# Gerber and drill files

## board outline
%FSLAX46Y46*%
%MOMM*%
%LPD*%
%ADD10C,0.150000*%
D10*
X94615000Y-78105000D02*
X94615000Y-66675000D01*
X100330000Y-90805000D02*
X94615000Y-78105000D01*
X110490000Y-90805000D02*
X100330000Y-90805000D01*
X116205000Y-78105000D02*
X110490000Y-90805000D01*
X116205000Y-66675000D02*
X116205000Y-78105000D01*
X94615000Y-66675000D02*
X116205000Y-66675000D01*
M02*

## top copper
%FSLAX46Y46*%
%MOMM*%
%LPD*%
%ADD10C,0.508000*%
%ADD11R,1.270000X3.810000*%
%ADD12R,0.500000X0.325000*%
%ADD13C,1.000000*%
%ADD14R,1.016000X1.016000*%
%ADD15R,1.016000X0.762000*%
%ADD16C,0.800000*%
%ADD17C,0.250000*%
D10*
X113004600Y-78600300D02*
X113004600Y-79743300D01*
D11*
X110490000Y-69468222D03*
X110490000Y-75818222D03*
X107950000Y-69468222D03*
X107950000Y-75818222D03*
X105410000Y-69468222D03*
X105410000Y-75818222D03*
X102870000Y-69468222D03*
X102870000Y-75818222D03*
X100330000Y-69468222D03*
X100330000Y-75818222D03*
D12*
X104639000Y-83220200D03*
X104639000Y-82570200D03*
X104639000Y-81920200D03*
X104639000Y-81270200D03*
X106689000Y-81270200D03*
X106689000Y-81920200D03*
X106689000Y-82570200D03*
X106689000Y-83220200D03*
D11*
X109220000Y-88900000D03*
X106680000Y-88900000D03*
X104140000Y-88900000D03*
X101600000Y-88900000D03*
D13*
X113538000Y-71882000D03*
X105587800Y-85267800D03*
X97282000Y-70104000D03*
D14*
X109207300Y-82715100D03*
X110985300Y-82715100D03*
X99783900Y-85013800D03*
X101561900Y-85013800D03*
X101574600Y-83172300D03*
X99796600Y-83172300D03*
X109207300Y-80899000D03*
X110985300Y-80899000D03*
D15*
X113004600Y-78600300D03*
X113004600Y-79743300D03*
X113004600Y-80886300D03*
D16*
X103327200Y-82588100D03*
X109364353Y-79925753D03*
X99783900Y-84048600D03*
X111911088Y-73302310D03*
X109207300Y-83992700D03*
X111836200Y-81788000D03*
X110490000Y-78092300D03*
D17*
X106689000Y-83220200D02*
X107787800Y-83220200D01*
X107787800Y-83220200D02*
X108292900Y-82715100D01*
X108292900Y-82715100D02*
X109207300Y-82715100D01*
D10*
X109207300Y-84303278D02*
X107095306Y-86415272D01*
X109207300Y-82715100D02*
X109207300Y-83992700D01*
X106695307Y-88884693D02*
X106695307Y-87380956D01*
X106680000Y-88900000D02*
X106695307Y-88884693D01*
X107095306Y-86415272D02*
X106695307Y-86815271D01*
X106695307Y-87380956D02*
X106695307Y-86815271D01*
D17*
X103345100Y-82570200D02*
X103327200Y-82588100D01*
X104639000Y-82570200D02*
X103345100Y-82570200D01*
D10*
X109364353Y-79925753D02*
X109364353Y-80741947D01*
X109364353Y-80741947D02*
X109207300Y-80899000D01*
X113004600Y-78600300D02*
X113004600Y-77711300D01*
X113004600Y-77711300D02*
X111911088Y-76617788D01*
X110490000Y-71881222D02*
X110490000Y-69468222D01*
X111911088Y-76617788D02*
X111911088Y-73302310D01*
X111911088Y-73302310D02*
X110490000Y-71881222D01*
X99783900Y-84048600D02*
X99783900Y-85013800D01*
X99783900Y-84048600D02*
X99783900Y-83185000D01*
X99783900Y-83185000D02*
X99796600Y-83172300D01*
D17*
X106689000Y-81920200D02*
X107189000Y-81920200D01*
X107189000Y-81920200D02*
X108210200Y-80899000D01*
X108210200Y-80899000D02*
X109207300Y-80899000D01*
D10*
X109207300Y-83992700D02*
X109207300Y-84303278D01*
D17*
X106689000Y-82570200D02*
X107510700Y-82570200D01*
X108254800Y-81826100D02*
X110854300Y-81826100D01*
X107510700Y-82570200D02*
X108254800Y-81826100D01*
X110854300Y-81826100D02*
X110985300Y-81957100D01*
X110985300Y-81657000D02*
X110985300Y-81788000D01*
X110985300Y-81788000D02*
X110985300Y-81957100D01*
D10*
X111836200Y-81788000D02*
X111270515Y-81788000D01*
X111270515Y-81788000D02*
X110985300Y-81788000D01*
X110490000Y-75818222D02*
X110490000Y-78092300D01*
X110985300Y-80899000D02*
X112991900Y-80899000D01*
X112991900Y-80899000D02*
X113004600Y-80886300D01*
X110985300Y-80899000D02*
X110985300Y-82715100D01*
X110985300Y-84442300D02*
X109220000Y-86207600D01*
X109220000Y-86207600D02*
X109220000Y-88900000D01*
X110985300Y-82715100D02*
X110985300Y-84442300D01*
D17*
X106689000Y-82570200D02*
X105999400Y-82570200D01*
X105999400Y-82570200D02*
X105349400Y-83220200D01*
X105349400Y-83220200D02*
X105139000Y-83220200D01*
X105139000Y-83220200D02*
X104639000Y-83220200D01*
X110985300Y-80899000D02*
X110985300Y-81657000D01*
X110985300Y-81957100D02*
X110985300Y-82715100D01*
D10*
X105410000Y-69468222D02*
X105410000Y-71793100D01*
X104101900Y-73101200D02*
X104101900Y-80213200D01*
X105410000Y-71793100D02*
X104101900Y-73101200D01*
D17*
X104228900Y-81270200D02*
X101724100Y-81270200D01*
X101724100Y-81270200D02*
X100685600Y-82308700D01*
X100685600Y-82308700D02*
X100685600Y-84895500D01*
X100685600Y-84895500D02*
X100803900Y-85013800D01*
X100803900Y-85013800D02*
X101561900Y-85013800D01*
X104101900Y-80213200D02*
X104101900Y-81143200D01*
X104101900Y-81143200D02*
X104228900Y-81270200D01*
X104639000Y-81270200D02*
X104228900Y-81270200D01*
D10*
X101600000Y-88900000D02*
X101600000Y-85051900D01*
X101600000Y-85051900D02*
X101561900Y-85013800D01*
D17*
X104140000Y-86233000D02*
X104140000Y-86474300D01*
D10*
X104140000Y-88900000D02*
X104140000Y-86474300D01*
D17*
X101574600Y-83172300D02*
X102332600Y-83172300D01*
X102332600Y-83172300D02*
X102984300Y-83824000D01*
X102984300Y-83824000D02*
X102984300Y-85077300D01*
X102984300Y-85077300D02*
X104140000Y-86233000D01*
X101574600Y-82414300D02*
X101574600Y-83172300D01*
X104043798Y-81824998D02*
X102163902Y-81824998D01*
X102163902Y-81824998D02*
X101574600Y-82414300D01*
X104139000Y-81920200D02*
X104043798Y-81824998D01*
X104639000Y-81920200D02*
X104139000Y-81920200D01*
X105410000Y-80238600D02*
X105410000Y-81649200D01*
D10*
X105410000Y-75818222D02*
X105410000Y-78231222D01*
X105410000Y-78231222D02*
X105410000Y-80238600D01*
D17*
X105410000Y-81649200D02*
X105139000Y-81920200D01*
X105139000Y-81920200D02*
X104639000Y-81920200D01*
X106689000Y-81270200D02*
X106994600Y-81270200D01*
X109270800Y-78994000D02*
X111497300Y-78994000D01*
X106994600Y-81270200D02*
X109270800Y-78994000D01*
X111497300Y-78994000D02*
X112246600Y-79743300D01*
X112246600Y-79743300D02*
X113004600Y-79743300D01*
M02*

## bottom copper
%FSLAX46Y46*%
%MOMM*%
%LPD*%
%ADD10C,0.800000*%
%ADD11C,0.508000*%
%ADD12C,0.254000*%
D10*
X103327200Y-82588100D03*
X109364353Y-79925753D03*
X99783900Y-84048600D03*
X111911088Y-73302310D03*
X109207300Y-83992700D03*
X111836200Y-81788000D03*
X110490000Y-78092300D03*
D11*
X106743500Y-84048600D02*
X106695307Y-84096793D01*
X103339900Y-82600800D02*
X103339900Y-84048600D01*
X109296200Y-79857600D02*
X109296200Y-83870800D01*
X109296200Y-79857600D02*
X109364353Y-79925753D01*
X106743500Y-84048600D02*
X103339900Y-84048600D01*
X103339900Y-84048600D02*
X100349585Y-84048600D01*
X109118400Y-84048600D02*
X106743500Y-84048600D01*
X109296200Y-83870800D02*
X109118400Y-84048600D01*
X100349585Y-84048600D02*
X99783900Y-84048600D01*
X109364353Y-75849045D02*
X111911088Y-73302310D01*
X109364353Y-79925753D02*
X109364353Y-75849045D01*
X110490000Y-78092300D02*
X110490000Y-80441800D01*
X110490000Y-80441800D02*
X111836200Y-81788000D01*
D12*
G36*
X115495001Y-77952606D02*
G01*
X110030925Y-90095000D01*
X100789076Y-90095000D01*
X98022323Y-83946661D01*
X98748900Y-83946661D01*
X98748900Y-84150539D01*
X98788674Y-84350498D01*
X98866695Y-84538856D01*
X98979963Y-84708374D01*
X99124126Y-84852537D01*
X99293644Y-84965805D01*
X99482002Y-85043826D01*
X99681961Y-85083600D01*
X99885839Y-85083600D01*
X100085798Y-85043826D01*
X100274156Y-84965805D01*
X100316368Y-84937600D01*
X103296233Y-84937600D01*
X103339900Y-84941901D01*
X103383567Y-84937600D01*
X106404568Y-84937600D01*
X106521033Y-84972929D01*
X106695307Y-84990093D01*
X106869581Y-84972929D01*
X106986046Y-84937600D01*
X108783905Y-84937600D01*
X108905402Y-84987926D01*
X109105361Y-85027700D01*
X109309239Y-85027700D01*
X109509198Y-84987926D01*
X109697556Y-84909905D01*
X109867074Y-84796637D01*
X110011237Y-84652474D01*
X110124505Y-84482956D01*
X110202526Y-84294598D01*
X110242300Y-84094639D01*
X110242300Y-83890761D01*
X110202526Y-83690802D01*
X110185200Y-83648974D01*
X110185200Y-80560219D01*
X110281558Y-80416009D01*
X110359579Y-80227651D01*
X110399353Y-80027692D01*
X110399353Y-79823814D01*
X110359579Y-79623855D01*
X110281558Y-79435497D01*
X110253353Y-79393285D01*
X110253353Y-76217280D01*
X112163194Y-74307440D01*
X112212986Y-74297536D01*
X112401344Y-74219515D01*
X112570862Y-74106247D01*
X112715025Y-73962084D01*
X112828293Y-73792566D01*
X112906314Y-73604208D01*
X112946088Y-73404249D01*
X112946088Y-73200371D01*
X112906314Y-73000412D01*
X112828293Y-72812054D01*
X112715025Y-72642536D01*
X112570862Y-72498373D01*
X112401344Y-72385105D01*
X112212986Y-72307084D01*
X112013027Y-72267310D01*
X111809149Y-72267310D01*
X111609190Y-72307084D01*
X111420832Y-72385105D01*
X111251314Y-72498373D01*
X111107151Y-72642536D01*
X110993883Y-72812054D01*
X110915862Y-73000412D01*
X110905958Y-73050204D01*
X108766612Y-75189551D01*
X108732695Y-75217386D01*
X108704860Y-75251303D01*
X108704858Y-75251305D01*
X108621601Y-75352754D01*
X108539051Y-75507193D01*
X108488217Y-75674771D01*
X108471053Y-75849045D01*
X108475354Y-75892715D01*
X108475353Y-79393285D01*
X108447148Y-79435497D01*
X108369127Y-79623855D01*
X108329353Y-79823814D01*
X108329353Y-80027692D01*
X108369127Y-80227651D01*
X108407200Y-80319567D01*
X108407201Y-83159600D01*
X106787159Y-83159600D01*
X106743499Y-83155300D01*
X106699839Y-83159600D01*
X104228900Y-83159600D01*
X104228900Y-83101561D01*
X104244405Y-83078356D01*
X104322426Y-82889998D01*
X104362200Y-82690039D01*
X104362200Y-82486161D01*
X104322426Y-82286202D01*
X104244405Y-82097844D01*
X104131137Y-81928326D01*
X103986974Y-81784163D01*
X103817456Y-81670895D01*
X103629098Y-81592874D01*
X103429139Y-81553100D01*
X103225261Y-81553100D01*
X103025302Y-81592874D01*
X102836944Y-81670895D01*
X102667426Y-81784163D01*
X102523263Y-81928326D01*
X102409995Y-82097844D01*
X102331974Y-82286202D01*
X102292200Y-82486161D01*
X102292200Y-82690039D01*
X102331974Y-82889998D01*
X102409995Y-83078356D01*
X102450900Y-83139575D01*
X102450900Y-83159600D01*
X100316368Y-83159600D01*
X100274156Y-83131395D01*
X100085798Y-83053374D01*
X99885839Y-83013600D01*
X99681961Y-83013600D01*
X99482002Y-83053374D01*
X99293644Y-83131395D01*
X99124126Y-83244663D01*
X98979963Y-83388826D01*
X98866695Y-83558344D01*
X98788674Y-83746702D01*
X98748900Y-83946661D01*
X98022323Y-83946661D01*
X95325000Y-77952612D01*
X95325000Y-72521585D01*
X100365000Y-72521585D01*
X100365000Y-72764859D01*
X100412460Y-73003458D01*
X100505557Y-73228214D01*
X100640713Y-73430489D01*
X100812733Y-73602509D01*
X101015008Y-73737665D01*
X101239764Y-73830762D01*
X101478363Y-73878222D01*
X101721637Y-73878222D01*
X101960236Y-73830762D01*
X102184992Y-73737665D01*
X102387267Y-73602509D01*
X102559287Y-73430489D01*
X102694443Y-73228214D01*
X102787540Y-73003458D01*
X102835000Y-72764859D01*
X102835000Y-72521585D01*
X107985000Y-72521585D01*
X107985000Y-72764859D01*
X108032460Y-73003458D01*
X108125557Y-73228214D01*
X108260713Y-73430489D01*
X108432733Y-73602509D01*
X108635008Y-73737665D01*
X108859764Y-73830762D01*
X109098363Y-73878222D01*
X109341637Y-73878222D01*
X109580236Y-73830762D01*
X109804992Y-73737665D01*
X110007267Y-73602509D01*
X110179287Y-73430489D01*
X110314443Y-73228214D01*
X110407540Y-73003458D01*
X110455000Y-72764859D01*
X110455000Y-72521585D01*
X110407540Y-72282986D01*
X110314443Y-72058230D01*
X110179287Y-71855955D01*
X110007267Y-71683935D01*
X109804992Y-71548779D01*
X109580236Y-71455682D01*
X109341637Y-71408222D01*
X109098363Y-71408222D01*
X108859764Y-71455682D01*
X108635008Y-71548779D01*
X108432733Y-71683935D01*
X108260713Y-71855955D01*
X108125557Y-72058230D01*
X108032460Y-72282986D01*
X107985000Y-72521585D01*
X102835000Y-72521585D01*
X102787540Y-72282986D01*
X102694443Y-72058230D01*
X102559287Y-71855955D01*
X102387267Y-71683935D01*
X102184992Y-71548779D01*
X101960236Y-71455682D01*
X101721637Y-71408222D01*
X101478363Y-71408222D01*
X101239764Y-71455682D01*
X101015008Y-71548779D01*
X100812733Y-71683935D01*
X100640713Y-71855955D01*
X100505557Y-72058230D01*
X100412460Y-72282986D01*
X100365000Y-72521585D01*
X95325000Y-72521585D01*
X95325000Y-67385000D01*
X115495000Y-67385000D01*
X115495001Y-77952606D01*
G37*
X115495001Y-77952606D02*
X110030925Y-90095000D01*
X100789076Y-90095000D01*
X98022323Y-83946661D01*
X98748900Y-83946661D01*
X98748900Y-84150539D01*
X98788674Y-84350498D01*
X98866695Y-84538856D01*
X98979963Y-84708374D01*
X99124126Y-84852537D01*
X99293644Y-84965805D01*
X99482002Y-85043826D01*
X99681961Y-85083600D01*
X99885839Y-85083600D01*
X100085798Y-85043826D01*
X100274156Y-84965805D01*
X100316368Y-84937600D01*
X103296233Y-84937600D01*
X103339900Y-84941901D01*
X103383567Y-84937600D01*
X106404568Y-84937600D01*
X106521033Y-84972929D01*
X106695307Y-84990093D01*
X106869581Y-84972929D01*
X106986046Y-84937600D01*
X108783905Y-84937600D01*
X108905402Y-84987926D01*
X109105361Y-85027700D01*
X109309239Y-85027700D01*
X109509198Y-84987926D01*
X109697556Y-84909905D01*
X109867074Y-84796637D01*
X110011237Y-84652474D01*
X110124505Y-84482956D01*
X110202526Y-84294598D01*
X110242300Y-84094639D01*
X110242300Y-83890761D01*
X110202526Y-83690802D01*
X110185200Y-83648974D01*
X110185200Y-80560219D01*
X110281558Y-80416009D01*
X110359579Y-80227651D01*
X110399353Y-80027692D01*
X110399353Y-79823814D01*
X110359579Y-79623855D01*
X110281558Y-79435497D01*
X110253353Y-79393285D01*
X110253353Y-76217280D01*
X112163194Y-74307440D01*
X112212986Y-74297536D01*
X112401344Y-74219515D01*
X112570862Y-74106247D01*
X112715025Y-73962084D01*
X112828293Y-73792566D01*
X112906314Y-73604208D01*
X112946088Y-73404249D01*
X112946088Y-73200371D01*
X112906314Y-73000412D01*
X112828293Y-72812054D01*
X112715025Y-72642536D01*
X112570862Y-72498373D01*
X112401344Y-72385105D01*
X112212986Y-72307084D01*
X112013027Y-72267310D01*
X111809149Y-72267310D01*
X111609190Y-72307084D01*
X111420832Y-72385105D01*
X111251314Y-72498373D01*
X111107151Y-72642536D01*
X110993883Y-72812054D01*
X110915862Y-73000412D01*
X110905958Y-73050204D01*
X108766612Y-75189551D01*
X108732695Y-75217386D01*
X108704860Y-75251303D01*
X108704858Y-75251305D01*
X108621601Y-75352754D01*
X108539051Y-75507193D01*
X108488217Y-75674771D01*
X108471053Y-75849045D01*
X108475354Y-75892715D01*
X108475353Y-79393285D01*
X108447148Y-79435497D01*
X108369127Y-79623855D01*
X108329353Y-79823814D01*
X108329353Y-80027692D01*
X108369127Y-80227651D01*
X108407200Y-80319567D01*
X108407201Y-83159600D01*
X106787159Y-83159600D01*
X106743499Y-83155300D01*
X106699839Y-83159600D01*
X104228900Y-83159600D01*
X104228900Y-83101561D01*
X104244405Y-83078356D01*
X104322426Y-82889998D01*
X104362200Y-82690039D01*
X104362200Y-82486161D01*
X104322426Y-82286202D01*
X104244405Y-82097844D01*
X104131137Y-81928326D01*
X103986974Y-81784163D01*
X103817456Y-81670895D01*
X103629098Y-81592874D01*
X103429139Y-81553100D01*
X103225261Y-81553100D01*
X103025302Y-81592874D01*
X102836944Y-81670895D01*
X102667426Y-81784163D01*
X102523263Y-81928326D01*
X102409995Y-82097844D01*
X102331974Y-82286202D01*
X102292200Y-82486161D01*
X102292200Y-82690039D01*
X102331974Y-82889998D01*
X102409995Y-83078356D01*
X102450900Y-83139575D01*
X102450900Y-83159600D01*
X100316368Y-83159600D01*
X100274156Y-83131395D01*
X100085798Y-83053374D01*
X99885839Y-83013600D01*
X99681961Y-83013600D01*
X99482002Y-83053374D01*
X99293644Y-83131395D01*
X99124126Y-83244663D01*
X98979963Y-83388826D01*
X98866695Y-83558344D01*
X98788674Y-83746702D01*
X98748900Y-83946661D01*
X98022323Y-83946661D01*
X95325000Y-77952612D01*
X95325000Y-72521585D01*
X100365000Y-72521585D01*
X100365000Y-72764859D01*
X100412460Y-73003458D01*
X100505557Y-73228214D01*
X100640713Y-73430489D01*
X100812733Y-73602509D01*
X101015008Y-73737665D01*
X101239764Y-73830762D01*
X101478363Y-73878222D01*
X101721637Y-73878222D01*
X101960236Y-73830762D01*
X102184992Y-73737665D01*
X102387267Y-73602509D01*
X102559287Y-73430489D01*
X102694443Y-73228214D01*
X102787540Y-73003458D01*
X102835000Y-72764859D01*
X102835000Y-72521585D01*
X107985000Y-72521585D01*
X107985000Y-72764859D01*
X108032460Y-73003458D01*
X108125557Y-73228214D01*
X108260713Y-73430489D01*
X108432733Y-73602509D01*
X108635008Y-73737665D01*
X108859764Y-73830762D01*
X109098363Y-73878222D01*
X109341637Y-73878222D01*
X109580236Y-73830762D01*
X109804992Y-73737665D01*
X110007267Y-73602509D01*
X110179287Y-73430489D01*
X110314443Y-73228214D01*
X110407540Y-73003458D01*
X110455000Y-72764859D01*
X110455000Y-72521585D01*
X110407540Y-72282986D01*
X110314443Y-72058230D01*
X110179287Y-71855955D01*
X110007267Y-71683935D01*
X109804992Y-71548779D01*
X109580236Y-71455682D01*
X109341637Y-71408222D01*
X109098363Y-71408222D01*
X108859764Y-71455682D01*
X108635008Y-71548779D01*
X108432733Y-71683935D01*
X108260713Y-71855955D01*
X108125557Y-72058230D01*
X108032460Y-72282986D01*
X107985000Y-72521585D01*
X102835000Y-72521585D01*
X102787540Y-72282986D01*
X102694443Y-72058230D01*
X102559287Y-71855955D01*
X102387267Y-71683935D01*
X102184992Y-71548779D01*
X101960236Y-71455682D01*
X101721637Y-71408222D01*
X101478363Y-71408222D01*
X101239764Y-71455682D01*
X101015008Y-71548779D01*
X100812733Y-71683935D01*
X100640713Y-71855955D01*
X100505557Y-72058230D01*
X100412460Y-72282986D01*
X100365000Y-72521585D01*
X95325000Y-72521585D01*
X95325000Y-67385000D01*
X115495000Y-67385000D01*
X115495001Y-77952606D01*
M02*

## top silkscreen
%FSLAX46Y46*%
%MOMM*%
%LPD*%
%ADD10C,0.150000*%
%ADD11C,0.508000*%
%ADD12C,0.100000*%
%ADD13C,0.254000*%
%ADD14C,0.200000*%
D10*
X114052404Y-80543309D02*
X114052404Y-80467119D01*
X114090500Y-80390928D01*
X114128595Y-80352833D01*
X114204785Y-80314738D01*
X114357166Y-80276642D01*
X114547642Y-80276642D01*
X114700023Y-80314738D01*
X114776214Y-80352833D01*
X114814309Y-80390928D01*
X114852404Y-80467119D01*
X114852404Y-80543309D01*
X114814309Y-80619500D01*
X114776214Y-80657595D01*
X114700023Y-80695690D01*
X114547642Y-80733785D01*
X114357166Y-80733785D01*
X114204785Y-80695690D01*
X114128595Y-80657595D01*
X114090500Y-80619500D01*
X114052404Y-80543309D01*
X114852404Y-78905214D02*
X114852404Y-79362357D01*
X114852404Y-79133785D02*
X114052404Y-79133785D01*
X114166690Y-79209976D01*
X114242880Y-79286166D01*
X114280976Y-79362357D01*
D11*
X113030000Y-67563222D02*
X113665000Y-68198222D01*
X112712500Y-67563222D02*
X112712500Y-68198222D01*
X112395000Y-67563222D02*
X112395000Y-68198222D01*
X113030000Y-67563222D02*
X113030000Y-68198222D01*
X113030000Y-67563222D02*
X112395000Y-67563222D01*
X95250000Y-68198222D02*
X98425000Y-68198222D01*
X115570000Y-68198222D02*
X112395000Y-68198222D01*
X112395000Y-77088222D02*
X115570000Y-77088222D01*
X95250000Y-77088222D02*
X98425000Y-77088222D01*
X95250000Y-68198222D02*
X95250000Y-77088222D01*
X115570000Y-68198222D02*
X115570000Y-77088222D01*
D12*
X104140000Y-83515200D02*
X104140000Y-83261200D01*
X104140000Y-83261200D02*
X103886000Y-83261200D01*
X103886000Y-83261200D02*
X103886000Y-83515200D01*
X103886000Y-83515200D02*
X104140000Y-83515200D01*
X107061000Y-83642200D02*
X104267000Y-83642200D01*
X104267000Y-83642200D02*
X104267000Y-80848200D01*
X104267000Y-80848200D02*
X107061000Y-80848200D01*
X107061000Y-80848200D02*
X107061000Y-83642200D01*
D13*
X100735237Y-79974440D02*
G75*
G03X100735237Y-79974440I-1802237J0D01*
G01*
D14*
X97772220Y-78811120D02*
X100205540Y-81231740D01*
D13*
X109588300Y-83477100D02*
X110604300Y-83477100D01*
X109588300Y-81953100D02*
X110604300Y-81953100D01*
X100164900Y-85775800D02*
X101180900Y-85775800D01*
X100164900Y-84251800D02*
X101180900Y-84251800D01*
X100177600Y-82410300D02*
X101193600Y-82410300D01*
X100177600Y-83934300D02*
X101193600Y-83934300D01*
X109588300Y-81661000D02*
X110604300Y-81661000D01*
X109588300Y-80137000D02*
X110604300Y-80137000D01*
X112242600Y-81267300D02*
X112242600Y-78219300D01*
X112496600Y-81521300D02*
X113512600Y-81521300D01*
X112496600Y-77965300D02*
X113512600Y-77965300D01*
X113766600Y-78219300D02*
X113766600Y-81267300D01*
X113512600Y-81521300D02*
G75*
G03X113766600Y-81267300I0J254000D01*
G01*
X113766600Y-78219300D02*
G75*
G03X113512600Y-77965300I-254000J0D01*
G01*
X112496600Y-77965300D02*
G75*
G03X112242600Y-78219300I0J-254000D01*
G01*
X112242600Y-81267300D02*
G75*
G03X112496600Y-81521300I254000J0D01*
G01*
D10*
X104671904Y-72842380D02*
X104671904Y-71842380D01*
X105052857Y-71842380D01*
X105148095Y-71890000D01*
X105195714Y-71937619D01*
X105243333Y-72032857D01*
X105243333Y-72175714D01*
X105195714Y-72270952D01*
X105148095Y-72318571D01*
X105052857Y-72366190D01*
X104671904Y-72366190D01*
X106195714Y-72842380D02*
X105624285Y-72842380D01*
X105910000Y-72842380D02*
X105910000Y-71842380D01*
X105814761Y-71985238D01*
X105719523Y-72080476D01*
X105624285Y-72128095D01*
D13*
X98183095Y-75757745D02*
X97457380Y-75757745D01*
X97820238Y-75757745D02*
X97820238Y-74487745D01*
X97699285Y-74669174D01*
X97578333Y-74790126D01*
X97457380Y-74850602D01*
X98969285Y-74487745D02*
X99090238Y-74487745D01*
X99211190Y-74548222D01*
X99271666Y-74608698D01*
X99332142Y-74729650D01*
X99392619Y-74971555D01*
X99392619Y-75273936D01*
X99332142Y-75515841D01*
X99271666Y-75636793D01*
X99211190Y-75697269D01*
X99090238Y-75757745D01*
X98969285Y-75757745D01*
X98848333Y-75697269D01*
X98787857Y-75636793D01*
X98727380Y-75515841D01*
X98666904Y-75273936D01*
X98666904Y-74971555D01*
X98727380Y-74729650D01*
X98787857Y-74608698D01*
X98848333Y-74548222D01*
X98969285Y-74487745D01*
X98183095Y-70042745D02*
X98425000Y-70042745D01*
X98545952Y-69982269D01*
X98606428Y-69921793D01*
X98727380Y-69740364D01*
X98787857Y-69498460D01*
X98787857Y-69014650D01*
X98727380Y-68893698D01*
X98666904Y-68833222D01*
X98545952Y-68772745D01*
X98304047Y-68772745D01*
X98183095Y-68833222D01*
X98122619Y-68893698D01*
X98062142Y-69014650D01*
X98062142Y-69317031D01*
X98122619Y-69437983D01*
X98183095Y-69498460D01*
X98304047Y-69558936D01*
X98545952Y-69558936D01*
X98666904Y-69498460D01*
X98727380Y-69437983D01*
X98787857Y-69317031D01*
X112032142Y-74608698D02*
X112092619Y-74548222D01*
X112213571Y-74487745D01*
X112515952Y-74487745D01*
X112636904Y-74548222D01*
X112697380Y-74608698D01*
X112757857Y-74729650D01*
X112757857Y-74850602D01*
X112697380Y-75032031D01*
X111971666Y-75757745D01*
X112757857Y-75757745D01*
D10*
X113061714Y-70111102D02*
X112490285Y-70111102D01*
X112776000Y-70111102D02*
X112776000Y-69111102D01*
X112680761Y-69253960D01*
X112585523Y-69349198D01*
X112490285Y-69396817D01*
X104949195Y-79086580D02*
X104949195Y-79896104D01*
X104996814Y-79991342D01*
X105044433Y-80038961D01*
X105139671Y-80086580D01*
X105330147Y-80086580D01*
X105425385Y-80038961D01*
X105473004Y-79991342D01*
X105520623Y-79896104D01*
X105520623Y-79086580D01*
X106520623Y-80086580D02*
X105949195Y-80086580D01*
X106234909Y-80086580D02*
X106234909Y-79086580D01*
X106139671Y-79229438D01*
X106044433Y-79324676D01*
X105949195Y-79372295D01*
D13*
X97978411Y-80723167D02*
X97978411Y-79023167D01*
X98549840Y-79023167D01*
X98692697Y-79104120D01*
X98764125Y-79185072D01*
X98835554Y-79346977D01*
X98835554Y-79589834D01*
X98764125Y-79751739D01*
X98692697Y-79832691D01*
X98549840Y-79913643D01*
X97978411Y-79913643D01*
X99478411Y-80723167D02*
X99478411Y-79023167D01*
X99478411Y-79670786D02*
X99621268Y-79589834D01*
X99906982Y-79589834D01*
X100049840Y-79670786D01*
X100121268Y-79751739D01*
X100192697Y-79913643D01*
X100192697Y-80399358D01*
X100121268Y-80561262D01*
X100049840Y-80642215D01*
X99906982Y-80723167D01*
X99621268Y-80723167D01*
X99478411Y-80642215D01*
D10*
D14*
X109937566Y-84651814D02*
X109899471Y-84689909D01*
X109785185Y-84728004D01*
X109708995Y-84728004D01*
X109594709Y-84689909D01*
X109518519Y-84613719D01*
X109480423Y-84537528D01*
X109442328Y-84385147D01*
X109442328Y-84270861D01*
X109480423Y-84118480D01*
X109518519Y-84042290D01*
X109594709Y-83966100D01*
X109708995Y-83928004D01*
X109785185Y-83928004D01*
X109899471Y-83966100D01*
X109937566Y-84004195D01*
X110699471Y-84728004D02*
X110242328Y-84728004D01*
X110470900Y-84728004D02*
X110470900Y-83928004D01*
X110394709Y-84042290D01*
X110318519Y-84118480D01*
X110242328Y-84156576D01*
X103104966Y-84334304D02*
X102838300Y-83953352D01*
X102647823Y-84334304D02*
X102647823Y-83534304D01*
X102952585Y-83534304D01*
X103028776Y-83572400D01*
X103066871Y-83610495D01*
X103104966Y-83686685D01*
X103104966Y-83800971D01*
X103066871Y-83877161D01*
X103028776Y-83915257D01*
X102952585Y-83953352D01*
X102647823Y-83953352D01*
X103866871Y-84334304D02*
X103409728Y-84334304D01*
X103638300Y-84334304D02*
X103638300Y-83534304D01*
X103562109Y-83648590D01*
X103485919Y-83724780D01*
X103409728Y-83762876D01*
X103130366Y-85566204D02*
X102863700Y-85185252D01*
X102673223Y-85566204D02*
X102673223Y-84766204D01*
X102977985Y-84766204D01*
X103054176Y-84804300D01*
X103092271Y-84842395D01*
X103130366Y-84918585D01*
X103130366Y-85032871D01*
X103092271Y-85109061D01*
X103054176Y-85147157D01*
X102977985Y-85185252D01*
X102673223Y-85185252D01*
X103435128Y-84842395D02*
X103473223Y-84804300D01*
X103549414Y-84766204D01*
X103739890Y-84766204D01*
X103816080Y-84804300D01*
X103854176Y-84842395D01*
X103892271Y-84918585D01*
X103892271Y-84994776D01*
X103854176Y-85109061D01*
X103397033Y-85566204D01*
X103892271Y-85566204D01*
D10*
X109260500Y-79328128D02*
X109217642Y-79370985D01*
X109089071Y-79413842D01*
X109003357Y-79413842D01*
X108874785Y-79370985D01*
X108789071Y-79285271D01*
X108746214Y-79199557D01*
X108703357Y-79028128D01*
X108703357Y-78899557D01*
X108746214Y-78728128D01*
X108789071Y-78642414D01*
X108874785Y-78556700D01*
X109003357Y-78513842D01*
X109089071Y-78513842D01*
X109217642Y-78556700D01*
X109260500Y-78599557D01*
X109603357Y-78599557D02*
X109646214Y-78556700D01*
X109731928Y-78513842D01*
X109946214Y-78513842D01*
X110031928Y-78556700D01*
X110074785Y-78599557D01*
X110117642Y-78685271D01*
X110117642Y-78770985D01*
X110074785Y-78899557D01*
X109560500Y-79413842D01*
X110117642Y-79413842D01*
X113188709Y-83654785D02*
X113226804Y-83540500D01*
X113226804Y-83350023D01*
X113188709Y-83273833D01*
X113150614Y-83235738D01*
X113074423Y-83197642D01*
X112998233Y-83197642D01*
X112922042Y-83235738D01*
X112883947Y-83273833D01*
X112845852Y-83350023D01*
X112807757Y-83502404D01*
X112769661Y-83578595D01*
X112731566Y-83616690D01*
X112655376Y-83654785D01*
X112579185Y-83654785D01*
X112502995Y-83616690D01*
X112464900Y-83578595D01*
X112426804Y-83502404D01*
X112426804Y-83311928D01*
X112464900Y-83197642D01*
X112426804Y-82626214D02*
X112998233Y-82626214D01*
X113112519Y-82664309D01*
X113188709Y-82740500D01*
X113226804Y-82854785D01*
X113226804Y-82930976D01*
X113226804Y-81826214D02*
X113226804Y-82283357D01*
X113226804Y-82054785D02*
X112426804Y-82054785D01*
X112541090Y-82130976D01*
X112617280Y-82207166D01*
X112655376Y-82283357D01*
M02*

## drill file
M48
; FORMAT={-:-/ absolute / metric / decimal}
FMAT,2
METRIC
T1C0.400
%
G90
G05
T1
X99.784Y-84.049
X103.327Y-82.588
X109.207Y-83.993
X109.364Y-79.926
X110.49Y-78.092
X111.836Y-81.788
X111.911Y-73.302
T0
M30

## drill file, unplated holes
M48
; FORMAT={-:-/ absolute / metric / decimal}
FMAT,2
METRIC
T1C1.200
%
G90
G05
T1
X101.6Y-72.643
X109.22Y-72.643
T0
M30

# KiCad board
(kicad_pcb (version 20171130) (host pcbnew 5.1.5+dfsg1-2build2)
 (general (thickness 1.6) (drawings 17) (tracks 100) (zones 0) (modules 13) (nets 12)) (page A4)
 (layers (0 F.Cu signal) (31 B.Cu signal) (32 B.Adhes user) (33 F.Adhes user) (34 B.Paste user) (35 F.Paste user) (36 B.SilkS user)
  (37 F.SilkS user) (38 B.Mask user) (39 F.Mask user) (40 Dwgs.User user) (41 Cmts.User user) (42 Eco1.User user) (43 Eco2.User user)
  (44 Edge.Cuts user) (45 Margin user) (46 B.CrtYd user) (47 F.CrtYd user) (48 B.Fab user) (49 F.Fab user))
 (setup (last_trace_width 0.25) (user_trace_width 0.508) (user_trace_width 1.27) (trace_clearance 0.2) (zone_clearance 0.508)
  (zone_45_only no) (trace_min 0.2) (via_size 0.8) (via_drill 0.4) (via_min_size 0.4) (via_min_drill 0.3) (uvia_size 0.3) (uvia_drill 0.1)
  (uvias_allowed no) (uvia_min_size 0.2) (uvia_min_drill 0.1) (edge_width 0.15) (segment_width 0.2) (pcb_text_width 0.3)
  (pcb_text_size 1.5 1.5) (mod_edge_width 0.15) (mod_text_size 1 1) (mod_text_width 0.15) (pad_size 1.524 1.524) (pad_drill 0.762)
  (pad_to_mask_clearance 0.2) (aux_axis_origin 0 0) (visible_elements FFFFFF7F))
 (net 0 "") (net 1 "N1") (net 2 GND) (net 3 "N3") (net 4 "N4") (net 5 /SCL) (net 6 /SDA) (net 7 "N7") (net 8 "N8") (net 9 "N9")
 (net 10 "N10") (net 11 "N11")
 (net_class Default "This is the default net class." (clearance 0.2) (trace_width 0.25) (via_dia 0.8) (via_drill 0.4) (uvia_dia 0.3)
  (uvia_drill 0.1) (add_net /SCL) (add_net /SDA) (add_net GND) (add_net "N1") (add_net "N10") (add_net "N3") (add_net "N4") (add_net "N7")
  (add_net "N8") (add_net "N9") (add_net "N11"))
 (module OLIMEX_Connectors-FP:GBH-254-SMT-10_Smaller (layer F.Cu) (at 105.41 72.643222) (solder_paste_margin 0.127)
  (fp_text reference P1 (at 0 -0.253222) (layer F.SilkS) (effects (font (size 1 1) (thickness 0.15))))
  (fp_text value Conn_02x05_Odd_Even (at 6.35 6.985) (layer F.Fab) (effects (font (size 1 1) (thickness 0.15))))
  (fp_line (start 7.62 -5.08) (end 8.255 -4.445) (layer F.SilkS) (width 0.508))
  (fp_line (start 7.3025 -5.08) (end 7.3025 -4.445) (layer F.SilkS) (width 0.508))
  (fp_line (start 6.985 -5.08) (end 6.985 -4.445) (layer F.SilkS) (width 0.508))
  (fp_line (start 7.62 -5.08) (end 7.62 -4.445) (layer F.SilkS) (width 0.508))
  (fp_line (start 7.62 -5.08) (end 6.985 -5.08) (layer F.SilkS) (width 0.508))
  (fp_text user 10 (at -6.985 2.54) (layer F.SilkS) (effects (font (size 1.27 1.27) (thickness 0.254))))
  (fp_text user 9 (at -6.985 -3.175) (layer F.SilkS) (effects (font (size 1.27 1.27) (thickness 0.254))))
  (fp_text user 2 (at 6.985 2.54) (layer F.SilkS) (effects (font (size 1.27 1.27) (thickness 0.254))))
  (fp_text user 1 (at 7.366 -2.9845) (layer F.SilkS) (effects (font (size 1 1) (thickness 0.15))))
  (fp_line (start -10.16 -4.445) (end -6.985 -4.445) (layer F.SilkS) (width 0.508))
  (fp_line (start 10.16 -4.445) (end 6.985 -4.445) (layer F.SilkS) (width 0.508))
  (fp_line (start 6.985 4.445) (end 10.16 4.445) (layer F.SilkS) (width 0.508))
  (fp_line (start -10.16 4.445) (end -6.985 4.445) (layer F.SilkS) (width 0.508))
  (fp_line (start -10.16 -4.445) (end -10.16 4.445) (layer F.SilkS) (width 0.508))
  (fp_line (start 10.16 -4.445) (end 10.16 4.445) (layer F.SilkS) (width 0.508))
  (pad 11 smd trapezoid (at 5.08 -3.175) (size 1.7 3.81) (layers F.Paste))
  (pad 11 smd trapezoid (at 2.54 -3.175) (size 1.7 3.81) (layers F.Paste))
  (pad 11 smd trapezoid (at 0 -3.175) (size 1.7 3.81) (layers F.Paste))
  (pad 11 smd trapezoid (at -2.54 -3.175) (size 1.7 3.81) (layers F.Paste))
  (pad 11 smd trapezoid (at -5.08 -3.175) (size 1.7 3.81) (layers F.Paste))
  (pad 1 smd rect (at 5.08 -3.175) (size 1.27 3.81) (layers F.Cu F.Mask) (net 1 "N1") (solder_mask_margin 0.0508)
   (solder_paste_margin 0.127) (clearance 0.0508))
  (pad 2 smd rect (at 5.08 3.175) (size 1.27 3.81) (layers F.Cu F.Mask) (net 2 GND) (solder_mask_margin 0.0508) (solder_paste_margin 0.127)
   (clearance 0.0508))
  (pad 3 smd rect (at 2.54 -3.175) (size 1.27 3.81) (layers F.Cu F.Mask) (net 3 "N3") (solder_mask_margin 0.0508)
   (solder_paste_margin 0.127) (clearance 0.0508))
  (pad 4 smd rect (at 2.54 3.175) (size 1.27 3.81) (layers F.Cu F.Mask) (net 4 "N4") (solder_mask_margin 0.0508) (solder_paste_margin 0.127)
   (clearance 0.0508))
  (pad 5 smd rect (at 0 -3.175) (size 1.27 3.81) (layers F.Cu F.Mask) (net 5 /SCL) (solder_mask_margin 0.0508) (solder_paste_margin 0.127)
   (clearance 0.0508))
  (pad 6 smd rect (at 0 3.175) (size 1.27 3.81) (layers F.Cu F.Mask) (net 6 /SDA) (solder_mask_margin 0.0508) (solder_paste_margin 0.127)
   (clearance 0.0508))
  (pad 7 smd rect (at -2.54 -3.175) (size 1.27 3.81) (layers F.Cu F.Mask) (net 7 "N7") (solder_mask_margin 0.0508)
   (solder_paste_margin 0.127) (clearance 0.0508))
  (pad 8 smd rect (at -2.54 3.175) (size 1.27 3.81) (layers F.Cu F.Mask) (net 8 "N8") (solder_mask_margin 0.0508)
   (solder_paste_margin 0.127) (clearance 0.0508))
  (pad 9 smd rect (at -5.08 -3.175) (size 1.27 3.81) (layers F.Cu F.Mask) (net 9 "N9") (solder_mask_margin 0.0508)
   (solder_paste_margin 0.127) (clearance 0.0508))
  (pad 10 smd rect (at -5.08 3.175) (size 1.27 3.81) (layers F.Cu F.Mask) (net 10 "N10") (solder_mask_margin 0.0508)
   (solder_paste_margin 0.127) (clearance 0.0508))
  (pad "" np_thru_hole circle (at -3.81 0) (size 1.2 1.2) (drill 1.2) (layers *.Cu *.Mask) (solder_mask_margin 0.0508))
  (pad "" np_thru_hole circle (at 3.81 0) (size 1.2 1.2) (drill 1.2) (layers *.Cu *.Mask) (solder_mask_margin 0.0508))
  (pad 11 smd trapezoid (at -5.08 3.175) (size 1.7 3.81) (layers F.Paste))
  (pad 11 smd trapezoid (at -2.54 3.175) (size 1.7 3.81) (layers F.Paste))
  (pad 11 smd trapezoid (at 0 3.175) (size 1.7 3.81) (layers F.Paste))
  (pad 11 smd trapezoid (at 2.54 3.175) (size 1.7 3.81) (layers F.Paste))
  (pad 11 smd trapezoid (at 5.08 3.175) (size 1.7 3.81) (layers F.Paste)))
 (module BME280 (layer F.Cu) (at 105.664 82.2452 180)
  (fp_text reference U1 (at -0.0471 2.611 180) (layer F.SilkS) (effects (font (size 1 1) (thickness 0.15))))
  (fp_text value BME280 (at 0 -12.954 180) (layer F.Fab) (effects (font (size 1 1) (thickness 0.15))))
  (fp_line (start 1.524 -1.27) (end 1.524 -1.016) (layer F.SilkS) (width 0.1))
  (fp_line (start 1.524 -1.016) (end 1.778 -1.016) (layer F.SilkS) (width 0.1))
  (fp_line (start 1.778 -1.016) (end 1.778 -1.27) (layer F.SilkS) (width 0.1))
  (fp_line (start 1.778 -1.27) (end 1.524 -1.27) (layer F.SilkS) (width 0.1))
  (fp_line (start -1.397 -1.397) (end 1.397 -1.397) (layer F.SilkS) (width 0.1))
  (fp_line (start 1.397 -1.397) (end 1.397 1.397) (layer F.SilkS) (width 0.1))
  (fp_line (start 1.397 1.397) (end -1.397 1.397) (layer F.SilkS) (width 0.1))
  (fp_line (start -1.397 1.397) (end -1.397 -1.397) (layer F.SilkS) (width 0.1))
  (pad 1 smd rect (at 1.025 -0.975 180) (size 0.5 0.325) (layers F.Cu F.Paste F.Mask) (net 2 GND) (solder_mask_margin 0.05))
  (pad 2 smd rect (at 1.025 -0.325 180) (size 0.5 0.325) (layers F.Cu F.Paste F.Mask) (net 1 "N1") (solder_mask_margin 0.05))
  (pad 3 smd rect (at 1.025 0.325 180) (size 0.5 0.325) (layers F.Cu F.Paste F.Mask) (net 6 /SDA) (solder_mask_margin 0.05))
  (pad 4 smd rect (at 1.025 0.975 180) (size 0.5 0.325) (layers F.Cu F.Paste F.Mask) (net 5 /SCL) (solder_mask_margin 0.05))
  (pad 5 smd rect (at -1.025 0.975 180) (size 0.5 0.325) (layers F.Cu F.Paste F.Mask) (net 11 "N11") (solder_mask_margin 0.05))
  (pad 6 smd rect (at -1.025 0.325 180) (size 0.5 0.325) (layers F.Cu F.Paste F.Mask) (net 1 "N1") (solder_mask_margin 0.05))
  (pad 7 smd rect (at -1.025 -0.325 180) (size 0.5 0.325) (layers F.Cu F.Paste F.Mask) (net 2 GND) (solder_mask_margin 0.05))
  (pad 8 smd rect (at -1.025 -0.975 180) (size 0.5 0.325) (layers F.Cu F.Paste F.Mask) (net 1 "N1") (solder_mask_margin 0.05)))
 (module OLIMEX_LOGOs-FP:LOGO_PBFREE (layer F.Cu) (at 99.1362 80.2894)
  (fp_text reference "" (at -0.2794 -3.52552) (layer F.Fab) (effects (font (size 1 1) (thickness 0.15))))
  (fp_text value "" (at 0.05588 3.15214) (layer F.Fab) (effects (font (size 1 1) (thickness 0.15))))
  (fp_circle (center -0.2032 -0.31496) (end 0.90678 -1.73482) (layer F.SilkS) (width 0.254))
  (fp_line (start -1.36398 -1.47828) (end 1.06934 0.94234) (layer F.SilkS) (width 0.2))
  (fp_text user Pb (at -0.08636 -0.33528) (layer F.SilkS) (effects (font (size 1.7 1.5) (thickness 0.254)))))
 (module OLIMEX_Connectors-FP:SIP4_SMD (layer F.Cu) (at 105.41 88.9 180)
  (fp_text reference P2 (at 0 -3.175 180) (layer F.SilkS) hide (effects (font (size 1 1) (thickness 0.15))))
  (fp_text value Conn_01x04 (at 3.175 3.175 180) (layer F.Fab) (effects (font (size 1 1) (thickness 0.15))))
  (pad 1 smd rect (at -3.81 0 180) (size 1.27 3.81) (layers F.Cu F.Mask) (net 2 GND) (solder_mask_margin 0.0508)
   (solder_paste_margin -0.0508) (clearance 0.0508))
  (pad 2 smd rect (at -1.27 0 180) (size 1.27 3.81) (layers F.Cu F.Mask) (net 1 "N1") (solder_mask_margin 0.0508)
   (solder_paste_margin -0.0508) (clearance 0.0508))
  (pad 3 smd rect (at 1.27 0 180) (size 1.27 3.81) (layers F.Cu F.Mask) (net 6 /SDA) (solder_mask_margin 0.0508)
   (solder_paste_margin -0.0508) (clearance 0.0508))
  (pad 4 smd rect (at 3.81 0 180) (size 1.27 3.81) (layers F.Cu F.Mask) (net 5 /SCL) (solder_mask_margin 0.0508)
   (solder_paste_margin -0.0508) (clearance 0.0508)))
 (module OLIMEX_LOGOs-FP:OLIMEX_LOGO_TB (layer B.Cu) (at 105.41 69.85 180)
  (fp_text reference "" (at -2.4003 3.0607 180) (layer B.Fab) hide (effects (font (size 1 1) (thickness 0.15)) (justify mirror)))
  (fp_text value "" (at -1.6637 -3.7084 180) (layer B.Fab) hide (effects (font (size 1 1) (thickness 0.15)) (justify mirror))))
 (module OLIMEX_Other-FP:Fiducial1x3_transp (layer F.Cu) (at 113.538 71.882)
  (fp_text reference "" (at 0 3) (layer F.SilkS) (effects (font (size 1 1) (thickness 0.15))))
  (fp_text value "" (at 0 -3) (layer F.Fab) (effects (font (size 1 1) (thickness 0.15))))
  (pad Fid1 connect circle (at 0 0) (size 1 1) (layers F.Cu F.Mask) (solder_mask_margin 0.127) (clearance 1.016) (zone_connect 0)))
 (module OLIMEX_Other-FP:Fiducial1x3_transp (layer F.Cu) (at 105.5878 85.2678)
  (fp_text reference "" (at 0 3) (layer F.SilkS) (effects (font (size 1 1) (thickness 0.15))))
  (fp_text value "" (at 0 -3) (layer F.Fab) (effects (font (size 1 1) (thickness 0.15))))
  (pad Fid1 connect circle (at 0 0) (size 1 1) (layers F.Cu F.Mask) (solder_mask_margin 0.127) (clearance 1.016) (zone_connect 0)))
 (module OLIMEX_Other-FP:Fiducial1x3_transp (layer F.Cu) (at 97.282 70.104)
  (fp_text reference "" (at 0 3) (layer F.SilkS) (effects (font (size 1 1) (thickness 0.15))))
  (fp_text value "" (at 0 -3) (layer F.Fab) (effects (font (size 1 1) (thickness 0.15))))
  (pad Fid1 connect circle (at 0 0) (size 1 1) (layers F.Cu F.Mask) (solder_mask_margin 0.127) (clearance 1.016) (zone_connect 0)))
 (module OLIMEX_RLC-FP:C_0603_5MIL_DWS (layer F.Cu) (at 110.0963 82.7151)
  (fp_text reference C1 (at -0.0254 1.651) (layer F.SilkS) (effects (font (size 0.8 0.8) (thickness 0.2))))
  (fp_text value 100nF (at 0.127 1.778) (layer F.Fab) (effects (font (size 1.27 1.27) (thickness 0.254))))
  (fp_line (start -0.508 0.762) (end 0.508 0.762) (layer F.SilkS) (width 0.254))
  (fp_line (start -0.508 -0.762) (end 0.508 -0.762) (layer F.SilkS) (width 0.254))
  (pad 1 smd rect (at -0.889 0) (size 1.016 1.016) (layers F.Cu F.Paste F.Mask) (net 1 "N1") (solder_mask_margin 0.0508) (clearance 0.0508))
  (pad 2 smd rect (at 0.889 0) (size 1.016 1.016) (layers F.Cu F.Paste F.Mask) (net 2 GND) (solder_mask_margin 0.0508) (clearance 0.0508)))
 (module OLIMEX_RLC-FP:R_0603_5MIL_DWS (layer F.Cu) (at 100.6729 85.0138)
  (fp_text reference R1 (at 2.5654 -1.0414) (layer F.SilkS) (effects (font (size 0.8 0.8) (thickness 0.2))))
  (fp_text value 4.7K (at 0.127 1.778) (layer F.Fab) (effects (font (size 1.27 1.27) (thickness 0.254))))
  (fp_line (start -0.508 0.762) (end 0.508 0.762) (layer F.SilkS) (width 0.254))
  (fp_line (start -0.508 -0.762) (end 0.508 -0.762) (layer F.SilkS) (width 0.254))
  (pad 1 smd rect (at -0.889 0) (size 1.016 1.016) (layers F.Cu F.Paste F.Mask) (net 1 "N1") (solder_mask_margin 0.0508))
  (pad 2 smd rect (at 0.889 0) (size 1.016 1.016) (layers F.Cu F.Paste F.Mask) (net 5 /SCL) (solder_mask_margin 0.0508)))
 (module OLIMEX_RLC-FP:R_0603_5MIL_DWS (layer F.Cu) (at 100.6856 83.1723)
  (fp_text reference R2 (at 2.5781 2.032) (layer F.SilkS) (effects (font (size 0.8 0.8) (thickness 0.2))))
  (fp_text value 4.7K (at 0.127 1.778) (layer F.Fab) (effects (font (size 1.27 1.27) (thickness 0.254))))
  (fp_line (start -0.508 -0.762) (end 0.508 -0.762) (layer F.SilkS) (width 0.254))
  (fp_line (start -0.508 0.762) (end 0.508 0.762) (layer F.SilkS) (width 0.254))
  (pad 2 smd rect (at 0.889 0) (size 1.016 1.016) (layers F.Cu F.Paste F.Mask) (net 6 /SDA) (solder_mask_margin 0.0508))
  (pad 1 smd rect (at -0.889 0) (size 1.016 1.016) (layers F.Cu F.Paste F.Mask) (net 1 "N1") (solder_mask_margin 0.0508)))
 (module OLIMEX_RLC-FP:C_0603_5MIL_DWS (layer F.Cu) (at 110.0963 80.899)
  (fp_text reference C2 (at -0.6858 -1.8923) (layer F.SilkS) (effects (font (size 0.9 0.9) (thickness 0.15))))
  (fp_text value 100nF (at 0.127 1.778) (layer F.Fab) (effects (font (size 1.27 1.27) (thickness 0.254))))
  (fp_line (start -0.508 0.762) (end 0.508 0.762) (layer F.SilkS) (width 0.254))
  (fp_line (start -0.508 -0.762) (end 0.508 -0.762) (layer F.SilkS) (width 0.254))
  (pad 1 smd rect (at -0.889 0) (size 1.016 1.016) (layers F.Cu F.Paste F.Mask) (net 1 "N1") (solder_mask_margin 0.0508) (clearance 0.0508))
  (pad 2 smd rect (at 0.889 0) (size 1.016 1.016) (layers F.Cu F.Paste F.Mask) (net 2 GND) (solder_mask_margin 0.0508) (clearance 0.0508)))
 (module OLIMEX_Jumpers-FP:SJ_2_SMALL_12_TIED (layer F.Cu) (at 113.0046 79.7433 270)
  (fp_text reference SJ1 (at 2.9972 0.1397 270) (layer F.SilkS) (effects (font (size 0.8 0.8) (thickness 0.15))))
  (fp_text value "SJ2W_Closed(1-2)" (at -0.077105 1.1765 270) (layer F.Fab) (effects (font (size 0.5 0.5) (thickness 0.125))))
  (fp_line (start 1.524 0.762) (end -1.524 0.762) (layer F.SilkS) (width 0.254))
  (fp_line (start 1.778 0.508) (end 1.778 -0.508) (layer F.SilkS) (width 0.254))
  (fp_line (start -1.778 0.508) (end -1.778 -0.508) (layer F.SilkS) (width 0.254))
  (fp_line (start -1.524 -0.762) (end 1.524 -0.762) (layer F.SilkS) (width 0.254))
  (fp_line (start -1.143 0) (end 0 0) (layer F.Cu) (width 0.508))
  (fp_arc (start 1.524 -0.508) (end 1.524 -0.762) (angle 90) (layer F.SilkS) (width 0.254))
  (fp_arc (start -1.524 -0.508) (end -1.778 -0.508) (angle 90) (layer F.SilkS) (width 0.254))
  (fp_arc (start -1.524 0.508) (end -1.524 0.762) (angle 90) (layer F.SilkS) (width 0.254))
  (fp_arc (start 1.524 0.508) (end 1.778 0.508) (angle 90) (layer F.SilkS) (width 0.254))
  (pad 1 smd rect (at -1.143 0 270) (size 0.762 1.016) (layers F.Cu F.Mask) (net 1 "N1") (solder_mask_margin 0.0508)
   (solder_paste_margin -0.0508) (clearance 0.0508))
  (pad 2 smd rect (at 0 0 270) (size 0.762 1.016) (layers F.Cu F.Mask) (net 11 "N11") (solder_mask_margin 0.0508)
   (solder_paste_margin -0.0508) (clearance 0.0508))
  (pad 3 smd rect (at 1.143 0 270) (size 0.762 1.016) (layers F.Cu F.Mask) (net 2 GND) (solder_mask_margin 0.0508)
   (solder_paste_margin -0.0508) (clearance 0.0508)))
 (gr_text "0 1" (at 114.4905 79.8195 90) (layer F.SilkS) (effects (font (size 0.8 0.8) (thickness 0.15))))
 (gr_line (start 94.615 78.105) (end 94.615 66.675) (layer Edge.Cuts) (width 0.15))
 (gr_line (start 100.33 90.805) (end 94.615 78.105) (layer Edge.Cuts) (width 0.15))
 (gr_line (start 110.49 90.805) (end 100.33 90.805) (layer Edge.Cuts) (width 0.15))
 (gr_line (start 116.205 78.105) (end 110.49 90.805) (layer Edge.Cuts) (width 0.15))
 (gr_line (start 116.205 66.675) (end 116.205 78.105) (layer Edge.Cuts) (width 0.15))
 (gr_line (start 94.615 66.675) (end 116.205 66.675) (layer Edge.Cuts) (width 0.15))
 (segment (start 106.689 83.2202) (end 107.7878 83.2202) (width 0.25) (layer F.Cu) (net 1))
 (segment (start 107.7878 83.2202) (end 108.2929 82.7151) (width 0.25) (layer F.Cu) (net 1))
 (segment (start 108.2929 82.7151) (end 109.2073 82.7151) (width 0.25) (layer F.Cu) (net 1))
 (segment (start 109.2073 84.303278) (end 107.095306 86.415272) (width 0.508) (layer F.Cu) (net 1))
 (segment (start 109.2073 82.7151) (end 109.2073 83.9927) (width 0.508) (layer F.Cu) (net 1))
 (segment (start 106.695307 88.884693) (end 106.695307 87.380956) (width 0.508) (layer F.Cu) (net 1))
 (segment (start 106.68 88.9) (end 106.695307 88.884693) (width 0.508) (layer F.Cu) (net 1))
 (segment (start 106.7435 84.0486) (end 106.695307 84.096793) (width 0.508) (layer B.Cu) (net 1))
 (segment (start 107.095306 86.415272) (end 106.695307 86.815271) (width 0.508) (layer F.Cu) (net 1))
 (segment (start 106.695307 87.380956) (end 106.695307 86.815271) (width 0.508) (layer F.Cu) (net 1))
 (segment (start 103.3451 82.5702) (end 103.3272 82.5881) (width 0.25) (layer F.Cu) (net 1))
 (segment (start 104.639 82.5702) (end 103.3451 82.5702) (width 0.25) (layer F.Cu) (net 1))
 (via (at 103.3272 82.5881) (size 0.8) (drill 0.4) (layers F.Cu B.Cu) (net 1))
 (segment (start 103.3399 82.6008) (end 103.3399 84.0486) (width 0.508) (layer B.Cu) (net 1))
 (segment (start 109.364353 79.925753) (end 109.364353 80.741947) (width 0.508) (layer F.Cu) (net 1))
 (segment (start 109.364353 80.741947) (end 109.2073 80.899) (width 0.508) (layer F.Cu) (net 1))
 (segment (start 109.2962 79.8576) (end 109.2962 83.8708) (width 0.508) (layer B.Cu) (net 1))
 (segment (start 109.2962 79.8576) (end 109.364353 79.925753) (width 0.508) (layer B.Cu) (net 1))
 (via (at 109.364353 79.925753) (size 0.8) (drill 0.4) (layers F.Cu B.Cu) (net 1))
 (segment (start 106.7435 84.0486) (end 103.3399 84.0486) (width 0.508) (layer B.Cu) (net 1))
 (segment (start 103.3399 84.0486) (end 100.349585 84.0486) (width 0.508) (layer B.Cu) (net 1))
 (segment (start 109.1184 84.0486) (end 106.7435 84.0486) (width 0.508) (layer B.Cu) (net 1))
 (segment (start 109.2962 83.8708) (end 109.1184 84.0486) (width 0.508) (layer B.Cu) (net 1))
 (segment (start 100.349585 84.0486) (end 99.7839 84.0486) (width 0.508) (layer B.Cu) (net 1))
 (segment (start 113.0046 78.6003) (end 113.0046 77.7113) (width 0.508) (layer F.Cu) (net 1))
 (segment (start 113.0046 77.7113) (end 111.911088 76.617788) (width 0.508) (layer F.Cu) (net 1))
 (segment (start 110.49 71.881222) (end 110.49 69.468222) (width 0.508) (layer F.Cu) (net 1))
 (segment (start 111.911088 76.617788) (end 111.911088 73.30231) (width 0.508) (layer F.Cu) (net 1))
 (segment (start 111.911088 73.30231) (end 110.49 71.881222) (width 0.508) (layer F.Cu) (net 1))
 (segment (start 99.7839 84.0486) (end 99.7839 85.0138) (width 0.508) (layer F.Cu) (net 1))
 (segment (start 99.7839 84.0486) (end 99.7839 83.185) (width 0.508) (layer F.Cu) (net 1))
 (segment (start 99.7839 83.185) (end 99.7966 83.1723) (width 0.508) (layer F.Cu) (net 1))
 (via (at 99.7839 84.0486) (size 0.8) (drill 0.4) (layers F.Cu B.Cu) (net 1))
 (segment (start 106.689 81.9202) (end 107.189 81.9202) (width 0.25) (layer F.Cu) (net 1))
 (segment (start 107.189 81.9202) (end 108.2102 80.899) (width 0.25) (layer F.Cu) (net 1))
 (segment (start 108.2102 80.899) (end 109.2073 80.899) (width 0.25) (layer F.Cu) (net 1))
 (via (at 111.911088 73.30231) (size 0.8) (drill 0.4) (layers F.Cu B.Cu) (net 1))
 (segment (start 109.364353 75.849045) (end 111.911088 73.30231) (width 0.508) (layer B.Cu) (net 1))
 (segment (start 109.364353 79.925753) (end 109.364353 75.849045) (width 0.508) (layer B.Cu) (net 1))
 (segment (start 109.2073 83.9927) (end 109.2073 84.303278) (width 0.508) (layer F.Cu) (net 1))
 (via (at 109.2073 83.9927) (size 0.8) (drill 0.4) (layers F.Cu B.Cu) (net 1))
 (segment (start 106.689 82.5702) (end 107.5107 82.5702) (width 0.25) (layer F.Cu) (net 2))
 (segment (start 108.2548 81.8261) (end 110.8543 81.8261) (width 0.25) (layer F.Cu) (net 2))
 (segment (start 107.5107 82.5702) (end 108.2548 81.8261) (width 0.25) (layer F.Cu) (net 2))
 (segment (start 110.8543 81.8261) (end 110.9853 81.9571) (width 0.25) (layer F.Cu) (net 2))
 (segment (start 110.9853 81.657) (end 110.9853 81.788) (width 0.25) (layer F.Cu) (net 2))
 (segment (start 110.9853 81.788) (end 110.9853 81.9571) (width 0.25) (layer F.Cu) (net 2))
 (segment (start 111.8362 81.788) (end 111.270515 81.788) (width 0.508) (layer F.Cu) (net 2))
 (segment (start 111.270515 81.788) (end 110.9853 81.788) (width 0.508) (layer F.Cu) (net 2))
 (segment (start 110.49 78.0923) (end 110.49 80.4418) (width 0.508) (layer B.Cu) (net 2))
 (segment (start 110.49 80.4418) (end 111.8362 81.788) (width 0.508) (layer B.Cu) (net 2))
 (via (at 111.8362 81.788) (size 0.8) (drill 0.4) (layers F.Cu B.Cu) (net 2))
 (segment (start 110.49 75.818222) (end 110.49 78.0923) (width 0.508) (layer F.Cu) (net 2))
 (via (at 110.49 78.0923) (size 0.8) (drill 0.4) (layers F.Cu B.Cu) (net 2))
 (segment (start 110.9853 80.899) (end 112.9919 80.899) (width 0.508) (layer F.Cu) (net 2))
 (segment (start 112.9919 80.899) (end 113.0046 80.8863) (width 0.508) (layer F.Cu) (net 2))
 (segment (start 110.9853 80.899) (end 110.9853 82.7151) (width 0.508) (layer F.Cu) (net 2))
 (segment (start 110.9853 84.4423) (end 109.22 86.2076) (width 0.508) (layer F.Cu) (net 2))
 (segment (start 109.22 86.2076) (end 109.22 88.9) (width 0.508) (layer F.Cu) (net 2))
 (segment (start 110.9853 82.7151) (end 110.9853 84.4423) (width 0.508) (layer F.Cu) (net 2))
 (segment (start 106.689 82.5702) (end 105.9994 82.5702) (width 0.25) (layer F.Cu) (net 2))
 (segment (start 105.9994 82.5702) (end 105.3494 83.2202) (width 0.25) (layer F.Cu) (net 2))
 (segment (start 105.3494 83.2202) (end 105.139 83.2202) (width 0.25) (layer F.Cu) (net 2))
 (segment (start 105.139 83.2202) (end 104.639 83.2202) (width 0.25) (layer F.Cu) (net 2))
 (segment (start 110.9853 80.899) (end 110.9853 81.657) (width 0.25) (layer F.Cu) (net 2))
 (segment (start 110.9853 81.9571) (end 110.9853 82.7151) (width 0.25) (layer F.Cu) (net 2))
 (segment (start 105.41 69.468222) (end 105.41 71.7931) (width 0.508) (layer F.Cu) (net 5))
 (segment (start 104.1019 73.1012) (end 104.1019 80.2132) (width 0.508) (layer F.Cu) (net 5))
 (segment (start 105.41 71.7931) (end 104.1019 73.1012) (width 0.508) (layer F.Cu) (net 5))
 (segment (start 104.2289 81.2702) (end 101.7241 81.2702) (width 0.25) (layer F.Cu) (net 5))
 (segment (start 101.7241 81.2702) (end 100.6856 82.3087) (width 0.25) (layer F.Cu) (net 5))
 (segment (start 100.6856 82.3087) (end 100.6856 84.8955) (width 0.25) (layer F.Cu) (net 5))
 (segment (start 100.6856 84.8955) (end 100.8039 85.0138) (width 0.25) (layer F.Cu) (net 5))
 (segment (start 100.8039 85.0138) (end 101.5619 85.0138) (width 0.25) (layer F.Cu) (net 5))
 (segment (start 104.1019 80.2132) (end 104.1019 81.1432) (width 0.25) (layer F.Cu) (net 5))
 (segment (start 104.1019 81.1432) (end 104.2289 81.2702) (width 0.25) (layer F.Cu) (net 5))
 (segment (start 104.639 81.2702) (end 104.2289 81.2702) (width 0.25) (layer F.Cu) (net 5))
 (segment (start 101.6 88.9) (end 101.6 85.0519) (width 0.508) (layer F.Cu) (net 5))
 (segment (start 101.6 85.0519) (end 101.5619 85.0138) (width 0.508) (layer F.Cu) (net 5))
 (segment (start 104.14 86.233) (end 104.14 86.4743) (width 0.25) (layer F.Cu) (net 6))
 (segment (start 104.14 88.9) (end 104.14 86.4743) (width 0.508) (layer F.Cu) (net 6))
 (segment (start 101.5746 83.1723) (end 102.3326 83.1723) (width 0.25) (layer F.Cu) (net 6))
 (segment (start 102.3326 83.1723) (end 102.9843 83.824) (width 0.25) (layer F.Cu) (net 6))
 (segment (start 102.9843 83.824) (end 102.9843 85.0773) (width 0.25) (layer F.Cu) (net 6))
 (segment (start 102.9843 85.0773) (end 104.14 86.233) (width 0.25) (layer F.Cu) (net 6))
 (segment (start 101.5746 82.4143) (end 101.5746 83.1723) (width 0.25) (layer F.Cu) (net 6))
 (segment (start 104.043798 81.824998) (end 102.163902 81.824998) (width 0.25) (layer F.Cu) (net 6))
 (segment (start 102.163902 81.824998) (end 101.5746 82.4143) (width 0.25) (layer F.Cu) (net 6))
 (segment (start 104.139 81.9202) (end 104.043798 81.824998) (width 0.25) (layer F.Cu) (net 6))
 (segment (start 104.639 81.9202) (end 104.139 81.9202) (width 0.25) (layer F.Cu) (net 6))
 (segment (start 105.41 80.2386) (end 105.41 81.6492) (width 0.25) (layer F.Cu) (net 6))
 (segment (start 105.41 75.818222) (end 105.41 78.231222) (width 0.508) (layer F.Cu) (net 6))
 (segment (start 105.41 78.231222) (end 105.41 80.2386) (width 0.508) (layer F.Cu) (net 6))
 (segment (start 105.41 81.6492) (end 105.139 81.9202) (width 0.25) (layer F.Cu) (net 6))
 (segment (start 105.139 81.9202) (end 104.639 81.9202) (width 0.25) (layer F.Cu) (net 6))
 (segment (start 106.689 81.2702) (end 106.9946 81.2702) (width 0.25) (layer F.Cu) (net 11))
 (segment (start 109.2708 78.994) (end 111.4973 78.994) (width 0.25) (layer F.Cu) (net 11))
 (segment (start 106.9946 81.2702) (end 109.2708 78.994) (width 0.25) (layer F.Cu) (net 11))
 (segment (start 111.4973 78.994) (end 112.2466 79.7433) (width 0.25) (layer F.Cu) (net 11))
 (segment (start 112.2466 79.7433) (end 113.0046 79.7433) (width 0.25) (layer F.Cu) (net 11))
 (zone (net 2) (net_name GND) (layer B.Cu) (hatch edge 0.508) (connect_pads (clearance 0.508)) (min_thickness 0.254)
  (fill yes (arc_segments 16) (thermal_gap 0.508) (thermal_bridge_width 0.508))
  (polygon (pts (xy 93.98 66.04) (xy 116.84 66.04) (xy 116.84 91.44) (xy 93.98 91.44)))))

